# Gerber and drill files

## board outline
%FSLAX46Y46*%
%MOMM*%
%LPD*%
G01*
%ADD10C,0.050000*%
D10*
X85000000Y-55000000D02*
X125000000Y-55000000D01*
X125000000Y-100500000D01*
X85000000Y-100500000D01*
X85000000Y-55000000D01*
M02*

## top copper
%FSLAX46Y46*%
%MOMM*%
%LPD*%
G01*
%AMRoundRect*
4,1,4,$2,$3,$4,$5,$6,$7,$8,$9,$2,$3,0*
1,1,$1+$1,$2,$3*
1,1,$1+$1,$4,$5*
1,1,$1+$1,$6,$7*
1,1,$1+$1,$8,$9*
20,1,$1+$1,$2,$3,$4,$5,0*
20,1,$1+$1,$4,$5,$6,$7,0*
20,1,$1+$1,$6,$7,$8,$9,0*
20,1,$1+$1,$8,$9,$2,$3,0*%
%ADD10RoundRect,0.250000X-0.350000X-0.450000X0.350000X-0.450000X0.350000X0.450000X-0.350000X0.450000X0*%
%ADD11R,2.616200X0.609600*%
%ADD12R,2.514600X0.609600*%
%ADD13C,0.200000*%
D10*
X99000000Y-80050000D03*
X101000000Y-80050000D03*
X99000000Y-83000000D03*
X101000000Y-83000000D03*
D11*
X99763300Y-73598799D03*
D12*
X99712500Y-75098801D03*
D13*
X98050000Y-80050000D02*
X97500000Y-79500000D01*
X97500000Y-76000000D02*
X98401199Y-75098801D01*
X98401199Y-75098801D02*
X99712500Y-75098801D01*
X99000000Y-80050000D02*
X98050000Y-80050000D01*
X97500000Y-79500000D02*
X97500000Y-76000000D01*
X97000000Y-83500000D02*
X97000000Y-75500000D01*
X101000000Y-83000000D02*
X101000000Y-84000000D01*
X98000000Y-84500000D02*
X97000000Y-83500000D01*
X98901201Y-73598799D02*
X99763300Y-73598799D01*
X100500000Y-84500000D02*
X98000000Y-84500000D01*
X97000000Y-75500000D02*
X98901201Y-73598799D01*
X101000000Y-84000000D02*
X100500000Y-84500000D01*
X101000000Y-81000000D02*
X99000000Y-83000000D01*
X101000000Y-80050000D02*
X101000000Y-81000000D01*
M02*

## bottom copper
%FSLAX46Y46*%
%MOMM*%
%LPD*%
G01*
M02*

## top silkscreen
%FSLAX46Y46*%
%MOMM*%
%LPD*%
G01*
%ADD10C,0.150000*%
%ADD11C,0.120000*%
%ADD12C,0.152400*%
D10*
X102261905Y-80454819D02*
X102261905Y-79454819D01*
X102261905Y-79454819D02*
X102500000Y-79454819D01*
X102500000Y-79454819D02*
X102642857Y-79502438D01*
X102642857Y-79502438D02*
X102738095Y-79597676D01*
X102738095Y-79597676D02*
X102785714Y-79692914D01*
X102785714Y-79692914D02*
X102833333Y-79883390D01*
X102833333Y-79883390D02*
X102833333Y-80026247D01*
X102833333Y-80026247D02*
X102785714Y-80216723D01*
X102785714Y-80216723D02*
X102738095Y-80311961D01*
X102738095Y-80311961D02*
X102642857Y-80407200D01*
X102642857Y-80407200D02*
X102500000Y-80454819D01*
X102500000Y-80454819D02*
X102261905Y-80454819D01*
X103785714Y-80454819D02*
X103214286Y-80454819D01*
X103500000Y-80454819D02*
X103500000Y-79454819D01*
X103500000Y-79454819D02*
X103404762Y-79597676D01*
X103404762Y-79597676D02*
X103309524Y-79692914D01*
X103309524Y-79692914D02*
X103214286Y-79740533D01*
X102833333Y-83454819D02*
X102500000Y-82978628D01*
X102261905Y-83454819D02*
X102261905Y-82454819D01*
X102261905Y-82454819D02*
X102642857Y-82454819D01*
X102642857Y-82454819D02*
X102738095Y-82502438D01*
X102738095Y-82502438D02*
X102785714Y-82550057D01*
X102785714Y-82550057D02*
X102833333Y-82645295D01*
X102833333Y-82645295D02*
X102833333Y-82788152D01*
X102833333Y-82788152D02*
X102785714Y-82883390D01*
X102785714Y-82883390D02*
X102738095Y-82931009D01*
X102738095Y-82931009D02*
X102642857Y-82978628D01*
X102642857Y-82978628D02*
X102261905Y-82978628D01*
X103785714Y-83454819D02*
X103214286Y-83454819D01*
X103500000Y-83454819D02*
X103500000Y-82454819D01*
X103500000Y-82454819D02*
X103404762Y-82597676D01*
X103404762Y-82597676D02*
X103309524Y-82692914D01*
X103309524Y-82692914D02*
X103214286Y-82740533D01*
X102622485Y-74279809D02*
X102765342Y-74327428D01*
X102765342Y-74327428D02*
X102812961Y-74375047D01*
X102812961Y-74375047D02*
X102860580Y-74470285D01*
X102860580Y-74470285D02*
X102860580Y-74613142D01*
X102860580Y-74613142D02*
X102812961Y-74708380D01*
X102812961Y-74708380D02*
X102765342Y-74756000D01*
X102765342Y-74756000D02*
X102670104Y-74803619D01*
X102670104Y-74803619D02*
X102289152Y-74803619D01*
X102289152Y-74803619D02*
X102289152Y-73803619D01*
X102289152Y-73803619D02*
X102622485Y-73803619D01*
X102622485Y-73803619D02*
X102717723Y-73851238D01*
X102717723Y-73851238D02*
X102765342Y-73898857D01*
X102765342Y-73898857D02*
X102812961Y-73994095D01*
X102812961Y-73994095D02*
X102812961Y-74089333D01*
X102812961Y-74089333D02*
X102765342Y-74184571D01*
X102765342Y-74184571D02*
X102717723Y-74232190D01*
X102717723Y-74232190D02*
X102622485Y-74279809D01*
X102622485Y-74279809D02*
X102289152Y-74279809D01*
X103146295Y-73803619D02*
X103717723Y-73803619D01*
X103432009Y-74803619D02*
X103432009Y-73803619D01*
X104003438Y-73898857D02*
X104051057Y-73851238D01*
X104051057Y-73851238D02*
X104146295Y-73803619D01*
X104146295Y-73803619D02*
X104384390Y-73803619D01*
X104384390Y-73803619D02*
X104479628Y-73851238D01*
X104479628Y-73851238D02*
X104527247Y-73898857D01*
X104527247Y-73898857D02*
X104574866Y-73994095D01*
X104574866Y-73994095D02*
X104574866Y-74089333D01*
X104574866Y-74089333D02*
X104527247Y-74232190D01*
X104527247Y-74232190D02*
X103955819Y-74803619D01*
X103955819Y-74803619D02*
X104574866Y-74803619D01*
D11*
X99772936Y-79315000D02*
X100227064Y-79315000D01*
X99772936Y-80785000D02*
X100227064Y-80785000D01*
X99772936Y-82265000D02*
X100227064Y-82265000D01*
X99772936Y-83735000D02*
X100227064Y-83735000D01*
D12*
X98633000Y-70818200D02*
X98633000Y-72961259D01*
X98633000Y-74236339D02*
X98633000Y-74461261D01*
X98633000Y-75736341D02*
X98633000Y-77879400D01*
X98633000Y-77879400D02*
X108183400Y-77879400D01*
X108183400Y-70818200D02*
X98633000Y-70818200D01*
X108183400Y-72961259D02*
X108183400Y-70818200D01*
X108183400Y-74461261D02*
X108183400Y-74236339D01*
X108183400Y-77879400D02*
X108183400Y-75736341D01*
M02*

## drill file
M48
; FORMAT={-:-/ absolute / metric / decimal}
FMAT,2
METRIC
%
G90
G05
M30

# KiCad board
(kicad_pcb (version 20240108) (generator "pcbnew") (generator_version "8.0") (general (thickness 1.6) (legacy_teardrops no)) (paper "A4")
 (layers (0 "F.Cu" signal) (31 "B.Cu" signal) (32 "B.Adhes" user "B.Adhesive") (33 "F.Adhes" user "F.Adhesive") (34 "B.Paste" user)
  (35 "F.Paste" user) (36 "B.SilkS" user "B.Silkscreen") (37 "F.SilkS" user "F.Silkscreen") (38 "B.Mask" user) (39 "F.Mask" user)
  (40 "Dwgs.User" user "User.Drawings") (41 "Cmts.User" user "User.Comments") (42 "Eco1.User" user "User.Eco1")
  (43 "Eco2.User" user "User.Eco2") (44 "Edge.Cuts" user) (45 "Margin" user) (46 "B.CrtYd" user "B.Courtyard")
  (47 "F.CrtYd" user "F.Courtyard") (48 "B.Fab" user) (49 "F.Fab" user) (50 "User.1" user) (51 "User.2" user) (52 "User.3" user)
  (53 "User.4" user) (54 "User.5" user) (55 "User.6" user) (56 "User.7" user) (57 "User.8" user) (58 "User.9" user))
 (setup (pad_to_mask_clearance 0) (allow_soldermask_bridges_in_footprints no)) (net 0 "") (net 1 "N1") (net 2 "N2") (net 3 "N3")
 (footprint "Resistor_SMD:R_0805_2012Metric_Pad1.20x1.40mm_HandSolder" (layer "F.Cu") (at 100 80.05)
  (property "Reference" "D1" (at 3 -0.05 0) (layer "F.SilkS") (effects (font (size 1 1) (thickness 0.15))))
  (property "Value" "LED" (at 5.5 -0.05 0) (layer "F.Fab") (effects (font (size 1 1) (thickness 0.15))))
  (fp_line (start -0.227064 -0.735) (end 0.227064 -0.735) (stroke (width 0.12) (type solid)) (layer "F.SilkS"))
  (fp_line (start -0.227064 0.735) (end 0.227064 0.735) (stroke (width 0.12) (type solid)) (layer "F.SilkS"))
  (pad "1" smd roundrect (at -1 0) (size 1.2 1.4) (layers "F.Cu" "F.Paste" "F.Mask") (roundrect_rratio 0.208333) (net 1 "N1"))
  (pad "2" smd roundrect (at 1 0) (size 1.2 1.4) (layers "F.Cu" "F.Paste" "F.Mask") (roundrect_rratio 0.208333) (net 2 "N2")))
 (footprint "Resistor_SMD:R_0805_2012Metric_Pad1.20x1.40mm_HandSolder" (layer "F.Cu") (at 100 83)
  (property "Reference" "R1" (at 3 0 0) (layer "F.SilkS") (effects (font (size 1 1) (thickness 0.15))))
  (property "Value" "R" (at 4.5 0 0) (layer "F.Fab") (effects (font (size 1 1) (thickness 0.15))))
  (fp_line (start -0.227064 -0.735) (end 0.227064 -0.735) (stroke (width 0.12) (type solid)) (layer "F.SilkS"))
  (fp_line (start -0.227064 0.735) (end 0.227064 0.735) (stroke (width 0.12) (type solid)) (layer "F.SilkS"))
  (pad "1" smd roundrect (at -1 0) (size 1.2 1.4) (layers "F.Cu" "F.Paste" "F.Mask") (roundrect_rratio 0.208333) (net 2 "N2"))
  (pad "2" smd roundrect (at 1 0) (size 1.2 1.4) (layers "F.Cu" "F.Paste" "F.Mask") (roundrect_rratio 0.208333) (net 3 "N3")))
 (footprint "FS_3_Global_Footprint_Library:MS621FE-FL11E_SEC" (layer "F.Cu") (at 103.4082 74.3488)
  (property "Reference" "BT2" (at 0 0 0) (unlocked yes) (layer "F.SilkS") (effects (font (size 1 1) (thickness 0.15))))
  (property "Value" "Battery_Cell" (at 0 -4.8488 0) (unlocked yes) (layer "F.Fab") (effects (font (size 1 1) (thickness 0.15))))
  (fp_line (start -4.7752 -3.5306) (end -4.7752 -1.387541) (stroke (width 0.1524) (type solid)) (layer "F.SilkS"))
  (fp_line (start -4.7752 -0.112461) (end -4.7752 0.112461) (stroke (width 0.1524) (type solid)) (layer "F.SilkS"))
  (fp_line (start -4.7752 1.387541) (end -4.7752 3.5306) (stroke (width 0.1524) (type solid)) (layer "F.SilkS"))
  (fp_line (start -4.7752 3.5306) (end 4.7752 3.5306) (stroke (width 0.1524) (type solid)) (layer "F.SilkS"))
  (fp_line (start 4.7752 -3.5306) (end -4.7752 -3.5306) (stroke (width 0.1524) (type solid)) (layer "F.SilkS"))
  (fp_line (start 4.7752 -1.387541) (end 4.7752 -3.5306) (stroke (width 0.1524) (type solid)) (layer "F.SilkS"))
  (fp_line (start 4.7752 0.112461) (end 4.7752 -0.112461) (stroke (width 0.1524) (type solid)) (layer "F.SilkS"))
  (fp_line (start 4.7752 3.5306) (end 4.7752 1.387541) (stroke (width 0.1524) (type solid)) (layer "F.SilkS"))
  (pad "1" smd rect (at -3.6449 -0.750001) (size 2.6162 0.6096) (layers "F.Cu" "F.Paste" "F.Mask") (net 3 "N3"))
  (pad "2" smd rect (at -3.6957 0.750001) (size 2.5146 0.6096) (layers "F.Cu" "F.Paste" "F.Mask") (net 1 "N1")))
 (gr_rect (start 85 55) (end 125 100.5) (stroke (width 0.05) (type default)) (fill none) (layer "Edge.Cuts"))
 (segment (start 98.05 80.05) (end 97.5 79.5) (width 0.2) (layer "F.Cu") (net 1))
 (segment (start 97.5 76) (end 98.401199 75.098801) (width 0.2) (layer "F.Cu") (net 1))
 (segment (start 98.401199 75.098801) (end 99.7125 75.098801) (width 0.2) (layer "F.Cu") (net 1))
 (segment (start 99 80.05) (end 98.05 80.05) (width 0.2) (layer "F.Cu") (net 1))
 (segment (start 97.5 79.5) (end 97.5 76) (width 0.2) (layer "F.Cu") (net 1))
 (segment (start 97 83.5) (end 97 75.5) (width 0.2) (layer "F.Cu") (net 3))
 (segment (start 101 83) (end 101 84) (width 0.2) (layer "F.Cu") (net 3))
 (segment (start 98 84.5) (end 97 83.5) (width 0.2) (layer "F.Cu") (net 3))
 (segment (start 98.901201 73.598799) (end 99.7633 73.598799) (width 0.2) (layer "F.Cu") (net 3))
 (segment (start 100.5 84.5) (end 98 84.5) (width 0.2) (layer "F.Cu") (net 3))
 (segment (start 97 75.5) (end 98.901201 73.598799) (width 0.2) (layer "F.Cu") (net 3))
 (segment (start 101 84) (end 100.5 84.5) (width 0.2) (layer "F.Cu") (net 3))
 (segment (start 101 81) (end 99 83) (width 0.2) (layer "F.Cu") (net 2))
 (segment (start 101 80.05) (end 101 81) (width 0.2) (layer "F.Cu") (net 2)))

